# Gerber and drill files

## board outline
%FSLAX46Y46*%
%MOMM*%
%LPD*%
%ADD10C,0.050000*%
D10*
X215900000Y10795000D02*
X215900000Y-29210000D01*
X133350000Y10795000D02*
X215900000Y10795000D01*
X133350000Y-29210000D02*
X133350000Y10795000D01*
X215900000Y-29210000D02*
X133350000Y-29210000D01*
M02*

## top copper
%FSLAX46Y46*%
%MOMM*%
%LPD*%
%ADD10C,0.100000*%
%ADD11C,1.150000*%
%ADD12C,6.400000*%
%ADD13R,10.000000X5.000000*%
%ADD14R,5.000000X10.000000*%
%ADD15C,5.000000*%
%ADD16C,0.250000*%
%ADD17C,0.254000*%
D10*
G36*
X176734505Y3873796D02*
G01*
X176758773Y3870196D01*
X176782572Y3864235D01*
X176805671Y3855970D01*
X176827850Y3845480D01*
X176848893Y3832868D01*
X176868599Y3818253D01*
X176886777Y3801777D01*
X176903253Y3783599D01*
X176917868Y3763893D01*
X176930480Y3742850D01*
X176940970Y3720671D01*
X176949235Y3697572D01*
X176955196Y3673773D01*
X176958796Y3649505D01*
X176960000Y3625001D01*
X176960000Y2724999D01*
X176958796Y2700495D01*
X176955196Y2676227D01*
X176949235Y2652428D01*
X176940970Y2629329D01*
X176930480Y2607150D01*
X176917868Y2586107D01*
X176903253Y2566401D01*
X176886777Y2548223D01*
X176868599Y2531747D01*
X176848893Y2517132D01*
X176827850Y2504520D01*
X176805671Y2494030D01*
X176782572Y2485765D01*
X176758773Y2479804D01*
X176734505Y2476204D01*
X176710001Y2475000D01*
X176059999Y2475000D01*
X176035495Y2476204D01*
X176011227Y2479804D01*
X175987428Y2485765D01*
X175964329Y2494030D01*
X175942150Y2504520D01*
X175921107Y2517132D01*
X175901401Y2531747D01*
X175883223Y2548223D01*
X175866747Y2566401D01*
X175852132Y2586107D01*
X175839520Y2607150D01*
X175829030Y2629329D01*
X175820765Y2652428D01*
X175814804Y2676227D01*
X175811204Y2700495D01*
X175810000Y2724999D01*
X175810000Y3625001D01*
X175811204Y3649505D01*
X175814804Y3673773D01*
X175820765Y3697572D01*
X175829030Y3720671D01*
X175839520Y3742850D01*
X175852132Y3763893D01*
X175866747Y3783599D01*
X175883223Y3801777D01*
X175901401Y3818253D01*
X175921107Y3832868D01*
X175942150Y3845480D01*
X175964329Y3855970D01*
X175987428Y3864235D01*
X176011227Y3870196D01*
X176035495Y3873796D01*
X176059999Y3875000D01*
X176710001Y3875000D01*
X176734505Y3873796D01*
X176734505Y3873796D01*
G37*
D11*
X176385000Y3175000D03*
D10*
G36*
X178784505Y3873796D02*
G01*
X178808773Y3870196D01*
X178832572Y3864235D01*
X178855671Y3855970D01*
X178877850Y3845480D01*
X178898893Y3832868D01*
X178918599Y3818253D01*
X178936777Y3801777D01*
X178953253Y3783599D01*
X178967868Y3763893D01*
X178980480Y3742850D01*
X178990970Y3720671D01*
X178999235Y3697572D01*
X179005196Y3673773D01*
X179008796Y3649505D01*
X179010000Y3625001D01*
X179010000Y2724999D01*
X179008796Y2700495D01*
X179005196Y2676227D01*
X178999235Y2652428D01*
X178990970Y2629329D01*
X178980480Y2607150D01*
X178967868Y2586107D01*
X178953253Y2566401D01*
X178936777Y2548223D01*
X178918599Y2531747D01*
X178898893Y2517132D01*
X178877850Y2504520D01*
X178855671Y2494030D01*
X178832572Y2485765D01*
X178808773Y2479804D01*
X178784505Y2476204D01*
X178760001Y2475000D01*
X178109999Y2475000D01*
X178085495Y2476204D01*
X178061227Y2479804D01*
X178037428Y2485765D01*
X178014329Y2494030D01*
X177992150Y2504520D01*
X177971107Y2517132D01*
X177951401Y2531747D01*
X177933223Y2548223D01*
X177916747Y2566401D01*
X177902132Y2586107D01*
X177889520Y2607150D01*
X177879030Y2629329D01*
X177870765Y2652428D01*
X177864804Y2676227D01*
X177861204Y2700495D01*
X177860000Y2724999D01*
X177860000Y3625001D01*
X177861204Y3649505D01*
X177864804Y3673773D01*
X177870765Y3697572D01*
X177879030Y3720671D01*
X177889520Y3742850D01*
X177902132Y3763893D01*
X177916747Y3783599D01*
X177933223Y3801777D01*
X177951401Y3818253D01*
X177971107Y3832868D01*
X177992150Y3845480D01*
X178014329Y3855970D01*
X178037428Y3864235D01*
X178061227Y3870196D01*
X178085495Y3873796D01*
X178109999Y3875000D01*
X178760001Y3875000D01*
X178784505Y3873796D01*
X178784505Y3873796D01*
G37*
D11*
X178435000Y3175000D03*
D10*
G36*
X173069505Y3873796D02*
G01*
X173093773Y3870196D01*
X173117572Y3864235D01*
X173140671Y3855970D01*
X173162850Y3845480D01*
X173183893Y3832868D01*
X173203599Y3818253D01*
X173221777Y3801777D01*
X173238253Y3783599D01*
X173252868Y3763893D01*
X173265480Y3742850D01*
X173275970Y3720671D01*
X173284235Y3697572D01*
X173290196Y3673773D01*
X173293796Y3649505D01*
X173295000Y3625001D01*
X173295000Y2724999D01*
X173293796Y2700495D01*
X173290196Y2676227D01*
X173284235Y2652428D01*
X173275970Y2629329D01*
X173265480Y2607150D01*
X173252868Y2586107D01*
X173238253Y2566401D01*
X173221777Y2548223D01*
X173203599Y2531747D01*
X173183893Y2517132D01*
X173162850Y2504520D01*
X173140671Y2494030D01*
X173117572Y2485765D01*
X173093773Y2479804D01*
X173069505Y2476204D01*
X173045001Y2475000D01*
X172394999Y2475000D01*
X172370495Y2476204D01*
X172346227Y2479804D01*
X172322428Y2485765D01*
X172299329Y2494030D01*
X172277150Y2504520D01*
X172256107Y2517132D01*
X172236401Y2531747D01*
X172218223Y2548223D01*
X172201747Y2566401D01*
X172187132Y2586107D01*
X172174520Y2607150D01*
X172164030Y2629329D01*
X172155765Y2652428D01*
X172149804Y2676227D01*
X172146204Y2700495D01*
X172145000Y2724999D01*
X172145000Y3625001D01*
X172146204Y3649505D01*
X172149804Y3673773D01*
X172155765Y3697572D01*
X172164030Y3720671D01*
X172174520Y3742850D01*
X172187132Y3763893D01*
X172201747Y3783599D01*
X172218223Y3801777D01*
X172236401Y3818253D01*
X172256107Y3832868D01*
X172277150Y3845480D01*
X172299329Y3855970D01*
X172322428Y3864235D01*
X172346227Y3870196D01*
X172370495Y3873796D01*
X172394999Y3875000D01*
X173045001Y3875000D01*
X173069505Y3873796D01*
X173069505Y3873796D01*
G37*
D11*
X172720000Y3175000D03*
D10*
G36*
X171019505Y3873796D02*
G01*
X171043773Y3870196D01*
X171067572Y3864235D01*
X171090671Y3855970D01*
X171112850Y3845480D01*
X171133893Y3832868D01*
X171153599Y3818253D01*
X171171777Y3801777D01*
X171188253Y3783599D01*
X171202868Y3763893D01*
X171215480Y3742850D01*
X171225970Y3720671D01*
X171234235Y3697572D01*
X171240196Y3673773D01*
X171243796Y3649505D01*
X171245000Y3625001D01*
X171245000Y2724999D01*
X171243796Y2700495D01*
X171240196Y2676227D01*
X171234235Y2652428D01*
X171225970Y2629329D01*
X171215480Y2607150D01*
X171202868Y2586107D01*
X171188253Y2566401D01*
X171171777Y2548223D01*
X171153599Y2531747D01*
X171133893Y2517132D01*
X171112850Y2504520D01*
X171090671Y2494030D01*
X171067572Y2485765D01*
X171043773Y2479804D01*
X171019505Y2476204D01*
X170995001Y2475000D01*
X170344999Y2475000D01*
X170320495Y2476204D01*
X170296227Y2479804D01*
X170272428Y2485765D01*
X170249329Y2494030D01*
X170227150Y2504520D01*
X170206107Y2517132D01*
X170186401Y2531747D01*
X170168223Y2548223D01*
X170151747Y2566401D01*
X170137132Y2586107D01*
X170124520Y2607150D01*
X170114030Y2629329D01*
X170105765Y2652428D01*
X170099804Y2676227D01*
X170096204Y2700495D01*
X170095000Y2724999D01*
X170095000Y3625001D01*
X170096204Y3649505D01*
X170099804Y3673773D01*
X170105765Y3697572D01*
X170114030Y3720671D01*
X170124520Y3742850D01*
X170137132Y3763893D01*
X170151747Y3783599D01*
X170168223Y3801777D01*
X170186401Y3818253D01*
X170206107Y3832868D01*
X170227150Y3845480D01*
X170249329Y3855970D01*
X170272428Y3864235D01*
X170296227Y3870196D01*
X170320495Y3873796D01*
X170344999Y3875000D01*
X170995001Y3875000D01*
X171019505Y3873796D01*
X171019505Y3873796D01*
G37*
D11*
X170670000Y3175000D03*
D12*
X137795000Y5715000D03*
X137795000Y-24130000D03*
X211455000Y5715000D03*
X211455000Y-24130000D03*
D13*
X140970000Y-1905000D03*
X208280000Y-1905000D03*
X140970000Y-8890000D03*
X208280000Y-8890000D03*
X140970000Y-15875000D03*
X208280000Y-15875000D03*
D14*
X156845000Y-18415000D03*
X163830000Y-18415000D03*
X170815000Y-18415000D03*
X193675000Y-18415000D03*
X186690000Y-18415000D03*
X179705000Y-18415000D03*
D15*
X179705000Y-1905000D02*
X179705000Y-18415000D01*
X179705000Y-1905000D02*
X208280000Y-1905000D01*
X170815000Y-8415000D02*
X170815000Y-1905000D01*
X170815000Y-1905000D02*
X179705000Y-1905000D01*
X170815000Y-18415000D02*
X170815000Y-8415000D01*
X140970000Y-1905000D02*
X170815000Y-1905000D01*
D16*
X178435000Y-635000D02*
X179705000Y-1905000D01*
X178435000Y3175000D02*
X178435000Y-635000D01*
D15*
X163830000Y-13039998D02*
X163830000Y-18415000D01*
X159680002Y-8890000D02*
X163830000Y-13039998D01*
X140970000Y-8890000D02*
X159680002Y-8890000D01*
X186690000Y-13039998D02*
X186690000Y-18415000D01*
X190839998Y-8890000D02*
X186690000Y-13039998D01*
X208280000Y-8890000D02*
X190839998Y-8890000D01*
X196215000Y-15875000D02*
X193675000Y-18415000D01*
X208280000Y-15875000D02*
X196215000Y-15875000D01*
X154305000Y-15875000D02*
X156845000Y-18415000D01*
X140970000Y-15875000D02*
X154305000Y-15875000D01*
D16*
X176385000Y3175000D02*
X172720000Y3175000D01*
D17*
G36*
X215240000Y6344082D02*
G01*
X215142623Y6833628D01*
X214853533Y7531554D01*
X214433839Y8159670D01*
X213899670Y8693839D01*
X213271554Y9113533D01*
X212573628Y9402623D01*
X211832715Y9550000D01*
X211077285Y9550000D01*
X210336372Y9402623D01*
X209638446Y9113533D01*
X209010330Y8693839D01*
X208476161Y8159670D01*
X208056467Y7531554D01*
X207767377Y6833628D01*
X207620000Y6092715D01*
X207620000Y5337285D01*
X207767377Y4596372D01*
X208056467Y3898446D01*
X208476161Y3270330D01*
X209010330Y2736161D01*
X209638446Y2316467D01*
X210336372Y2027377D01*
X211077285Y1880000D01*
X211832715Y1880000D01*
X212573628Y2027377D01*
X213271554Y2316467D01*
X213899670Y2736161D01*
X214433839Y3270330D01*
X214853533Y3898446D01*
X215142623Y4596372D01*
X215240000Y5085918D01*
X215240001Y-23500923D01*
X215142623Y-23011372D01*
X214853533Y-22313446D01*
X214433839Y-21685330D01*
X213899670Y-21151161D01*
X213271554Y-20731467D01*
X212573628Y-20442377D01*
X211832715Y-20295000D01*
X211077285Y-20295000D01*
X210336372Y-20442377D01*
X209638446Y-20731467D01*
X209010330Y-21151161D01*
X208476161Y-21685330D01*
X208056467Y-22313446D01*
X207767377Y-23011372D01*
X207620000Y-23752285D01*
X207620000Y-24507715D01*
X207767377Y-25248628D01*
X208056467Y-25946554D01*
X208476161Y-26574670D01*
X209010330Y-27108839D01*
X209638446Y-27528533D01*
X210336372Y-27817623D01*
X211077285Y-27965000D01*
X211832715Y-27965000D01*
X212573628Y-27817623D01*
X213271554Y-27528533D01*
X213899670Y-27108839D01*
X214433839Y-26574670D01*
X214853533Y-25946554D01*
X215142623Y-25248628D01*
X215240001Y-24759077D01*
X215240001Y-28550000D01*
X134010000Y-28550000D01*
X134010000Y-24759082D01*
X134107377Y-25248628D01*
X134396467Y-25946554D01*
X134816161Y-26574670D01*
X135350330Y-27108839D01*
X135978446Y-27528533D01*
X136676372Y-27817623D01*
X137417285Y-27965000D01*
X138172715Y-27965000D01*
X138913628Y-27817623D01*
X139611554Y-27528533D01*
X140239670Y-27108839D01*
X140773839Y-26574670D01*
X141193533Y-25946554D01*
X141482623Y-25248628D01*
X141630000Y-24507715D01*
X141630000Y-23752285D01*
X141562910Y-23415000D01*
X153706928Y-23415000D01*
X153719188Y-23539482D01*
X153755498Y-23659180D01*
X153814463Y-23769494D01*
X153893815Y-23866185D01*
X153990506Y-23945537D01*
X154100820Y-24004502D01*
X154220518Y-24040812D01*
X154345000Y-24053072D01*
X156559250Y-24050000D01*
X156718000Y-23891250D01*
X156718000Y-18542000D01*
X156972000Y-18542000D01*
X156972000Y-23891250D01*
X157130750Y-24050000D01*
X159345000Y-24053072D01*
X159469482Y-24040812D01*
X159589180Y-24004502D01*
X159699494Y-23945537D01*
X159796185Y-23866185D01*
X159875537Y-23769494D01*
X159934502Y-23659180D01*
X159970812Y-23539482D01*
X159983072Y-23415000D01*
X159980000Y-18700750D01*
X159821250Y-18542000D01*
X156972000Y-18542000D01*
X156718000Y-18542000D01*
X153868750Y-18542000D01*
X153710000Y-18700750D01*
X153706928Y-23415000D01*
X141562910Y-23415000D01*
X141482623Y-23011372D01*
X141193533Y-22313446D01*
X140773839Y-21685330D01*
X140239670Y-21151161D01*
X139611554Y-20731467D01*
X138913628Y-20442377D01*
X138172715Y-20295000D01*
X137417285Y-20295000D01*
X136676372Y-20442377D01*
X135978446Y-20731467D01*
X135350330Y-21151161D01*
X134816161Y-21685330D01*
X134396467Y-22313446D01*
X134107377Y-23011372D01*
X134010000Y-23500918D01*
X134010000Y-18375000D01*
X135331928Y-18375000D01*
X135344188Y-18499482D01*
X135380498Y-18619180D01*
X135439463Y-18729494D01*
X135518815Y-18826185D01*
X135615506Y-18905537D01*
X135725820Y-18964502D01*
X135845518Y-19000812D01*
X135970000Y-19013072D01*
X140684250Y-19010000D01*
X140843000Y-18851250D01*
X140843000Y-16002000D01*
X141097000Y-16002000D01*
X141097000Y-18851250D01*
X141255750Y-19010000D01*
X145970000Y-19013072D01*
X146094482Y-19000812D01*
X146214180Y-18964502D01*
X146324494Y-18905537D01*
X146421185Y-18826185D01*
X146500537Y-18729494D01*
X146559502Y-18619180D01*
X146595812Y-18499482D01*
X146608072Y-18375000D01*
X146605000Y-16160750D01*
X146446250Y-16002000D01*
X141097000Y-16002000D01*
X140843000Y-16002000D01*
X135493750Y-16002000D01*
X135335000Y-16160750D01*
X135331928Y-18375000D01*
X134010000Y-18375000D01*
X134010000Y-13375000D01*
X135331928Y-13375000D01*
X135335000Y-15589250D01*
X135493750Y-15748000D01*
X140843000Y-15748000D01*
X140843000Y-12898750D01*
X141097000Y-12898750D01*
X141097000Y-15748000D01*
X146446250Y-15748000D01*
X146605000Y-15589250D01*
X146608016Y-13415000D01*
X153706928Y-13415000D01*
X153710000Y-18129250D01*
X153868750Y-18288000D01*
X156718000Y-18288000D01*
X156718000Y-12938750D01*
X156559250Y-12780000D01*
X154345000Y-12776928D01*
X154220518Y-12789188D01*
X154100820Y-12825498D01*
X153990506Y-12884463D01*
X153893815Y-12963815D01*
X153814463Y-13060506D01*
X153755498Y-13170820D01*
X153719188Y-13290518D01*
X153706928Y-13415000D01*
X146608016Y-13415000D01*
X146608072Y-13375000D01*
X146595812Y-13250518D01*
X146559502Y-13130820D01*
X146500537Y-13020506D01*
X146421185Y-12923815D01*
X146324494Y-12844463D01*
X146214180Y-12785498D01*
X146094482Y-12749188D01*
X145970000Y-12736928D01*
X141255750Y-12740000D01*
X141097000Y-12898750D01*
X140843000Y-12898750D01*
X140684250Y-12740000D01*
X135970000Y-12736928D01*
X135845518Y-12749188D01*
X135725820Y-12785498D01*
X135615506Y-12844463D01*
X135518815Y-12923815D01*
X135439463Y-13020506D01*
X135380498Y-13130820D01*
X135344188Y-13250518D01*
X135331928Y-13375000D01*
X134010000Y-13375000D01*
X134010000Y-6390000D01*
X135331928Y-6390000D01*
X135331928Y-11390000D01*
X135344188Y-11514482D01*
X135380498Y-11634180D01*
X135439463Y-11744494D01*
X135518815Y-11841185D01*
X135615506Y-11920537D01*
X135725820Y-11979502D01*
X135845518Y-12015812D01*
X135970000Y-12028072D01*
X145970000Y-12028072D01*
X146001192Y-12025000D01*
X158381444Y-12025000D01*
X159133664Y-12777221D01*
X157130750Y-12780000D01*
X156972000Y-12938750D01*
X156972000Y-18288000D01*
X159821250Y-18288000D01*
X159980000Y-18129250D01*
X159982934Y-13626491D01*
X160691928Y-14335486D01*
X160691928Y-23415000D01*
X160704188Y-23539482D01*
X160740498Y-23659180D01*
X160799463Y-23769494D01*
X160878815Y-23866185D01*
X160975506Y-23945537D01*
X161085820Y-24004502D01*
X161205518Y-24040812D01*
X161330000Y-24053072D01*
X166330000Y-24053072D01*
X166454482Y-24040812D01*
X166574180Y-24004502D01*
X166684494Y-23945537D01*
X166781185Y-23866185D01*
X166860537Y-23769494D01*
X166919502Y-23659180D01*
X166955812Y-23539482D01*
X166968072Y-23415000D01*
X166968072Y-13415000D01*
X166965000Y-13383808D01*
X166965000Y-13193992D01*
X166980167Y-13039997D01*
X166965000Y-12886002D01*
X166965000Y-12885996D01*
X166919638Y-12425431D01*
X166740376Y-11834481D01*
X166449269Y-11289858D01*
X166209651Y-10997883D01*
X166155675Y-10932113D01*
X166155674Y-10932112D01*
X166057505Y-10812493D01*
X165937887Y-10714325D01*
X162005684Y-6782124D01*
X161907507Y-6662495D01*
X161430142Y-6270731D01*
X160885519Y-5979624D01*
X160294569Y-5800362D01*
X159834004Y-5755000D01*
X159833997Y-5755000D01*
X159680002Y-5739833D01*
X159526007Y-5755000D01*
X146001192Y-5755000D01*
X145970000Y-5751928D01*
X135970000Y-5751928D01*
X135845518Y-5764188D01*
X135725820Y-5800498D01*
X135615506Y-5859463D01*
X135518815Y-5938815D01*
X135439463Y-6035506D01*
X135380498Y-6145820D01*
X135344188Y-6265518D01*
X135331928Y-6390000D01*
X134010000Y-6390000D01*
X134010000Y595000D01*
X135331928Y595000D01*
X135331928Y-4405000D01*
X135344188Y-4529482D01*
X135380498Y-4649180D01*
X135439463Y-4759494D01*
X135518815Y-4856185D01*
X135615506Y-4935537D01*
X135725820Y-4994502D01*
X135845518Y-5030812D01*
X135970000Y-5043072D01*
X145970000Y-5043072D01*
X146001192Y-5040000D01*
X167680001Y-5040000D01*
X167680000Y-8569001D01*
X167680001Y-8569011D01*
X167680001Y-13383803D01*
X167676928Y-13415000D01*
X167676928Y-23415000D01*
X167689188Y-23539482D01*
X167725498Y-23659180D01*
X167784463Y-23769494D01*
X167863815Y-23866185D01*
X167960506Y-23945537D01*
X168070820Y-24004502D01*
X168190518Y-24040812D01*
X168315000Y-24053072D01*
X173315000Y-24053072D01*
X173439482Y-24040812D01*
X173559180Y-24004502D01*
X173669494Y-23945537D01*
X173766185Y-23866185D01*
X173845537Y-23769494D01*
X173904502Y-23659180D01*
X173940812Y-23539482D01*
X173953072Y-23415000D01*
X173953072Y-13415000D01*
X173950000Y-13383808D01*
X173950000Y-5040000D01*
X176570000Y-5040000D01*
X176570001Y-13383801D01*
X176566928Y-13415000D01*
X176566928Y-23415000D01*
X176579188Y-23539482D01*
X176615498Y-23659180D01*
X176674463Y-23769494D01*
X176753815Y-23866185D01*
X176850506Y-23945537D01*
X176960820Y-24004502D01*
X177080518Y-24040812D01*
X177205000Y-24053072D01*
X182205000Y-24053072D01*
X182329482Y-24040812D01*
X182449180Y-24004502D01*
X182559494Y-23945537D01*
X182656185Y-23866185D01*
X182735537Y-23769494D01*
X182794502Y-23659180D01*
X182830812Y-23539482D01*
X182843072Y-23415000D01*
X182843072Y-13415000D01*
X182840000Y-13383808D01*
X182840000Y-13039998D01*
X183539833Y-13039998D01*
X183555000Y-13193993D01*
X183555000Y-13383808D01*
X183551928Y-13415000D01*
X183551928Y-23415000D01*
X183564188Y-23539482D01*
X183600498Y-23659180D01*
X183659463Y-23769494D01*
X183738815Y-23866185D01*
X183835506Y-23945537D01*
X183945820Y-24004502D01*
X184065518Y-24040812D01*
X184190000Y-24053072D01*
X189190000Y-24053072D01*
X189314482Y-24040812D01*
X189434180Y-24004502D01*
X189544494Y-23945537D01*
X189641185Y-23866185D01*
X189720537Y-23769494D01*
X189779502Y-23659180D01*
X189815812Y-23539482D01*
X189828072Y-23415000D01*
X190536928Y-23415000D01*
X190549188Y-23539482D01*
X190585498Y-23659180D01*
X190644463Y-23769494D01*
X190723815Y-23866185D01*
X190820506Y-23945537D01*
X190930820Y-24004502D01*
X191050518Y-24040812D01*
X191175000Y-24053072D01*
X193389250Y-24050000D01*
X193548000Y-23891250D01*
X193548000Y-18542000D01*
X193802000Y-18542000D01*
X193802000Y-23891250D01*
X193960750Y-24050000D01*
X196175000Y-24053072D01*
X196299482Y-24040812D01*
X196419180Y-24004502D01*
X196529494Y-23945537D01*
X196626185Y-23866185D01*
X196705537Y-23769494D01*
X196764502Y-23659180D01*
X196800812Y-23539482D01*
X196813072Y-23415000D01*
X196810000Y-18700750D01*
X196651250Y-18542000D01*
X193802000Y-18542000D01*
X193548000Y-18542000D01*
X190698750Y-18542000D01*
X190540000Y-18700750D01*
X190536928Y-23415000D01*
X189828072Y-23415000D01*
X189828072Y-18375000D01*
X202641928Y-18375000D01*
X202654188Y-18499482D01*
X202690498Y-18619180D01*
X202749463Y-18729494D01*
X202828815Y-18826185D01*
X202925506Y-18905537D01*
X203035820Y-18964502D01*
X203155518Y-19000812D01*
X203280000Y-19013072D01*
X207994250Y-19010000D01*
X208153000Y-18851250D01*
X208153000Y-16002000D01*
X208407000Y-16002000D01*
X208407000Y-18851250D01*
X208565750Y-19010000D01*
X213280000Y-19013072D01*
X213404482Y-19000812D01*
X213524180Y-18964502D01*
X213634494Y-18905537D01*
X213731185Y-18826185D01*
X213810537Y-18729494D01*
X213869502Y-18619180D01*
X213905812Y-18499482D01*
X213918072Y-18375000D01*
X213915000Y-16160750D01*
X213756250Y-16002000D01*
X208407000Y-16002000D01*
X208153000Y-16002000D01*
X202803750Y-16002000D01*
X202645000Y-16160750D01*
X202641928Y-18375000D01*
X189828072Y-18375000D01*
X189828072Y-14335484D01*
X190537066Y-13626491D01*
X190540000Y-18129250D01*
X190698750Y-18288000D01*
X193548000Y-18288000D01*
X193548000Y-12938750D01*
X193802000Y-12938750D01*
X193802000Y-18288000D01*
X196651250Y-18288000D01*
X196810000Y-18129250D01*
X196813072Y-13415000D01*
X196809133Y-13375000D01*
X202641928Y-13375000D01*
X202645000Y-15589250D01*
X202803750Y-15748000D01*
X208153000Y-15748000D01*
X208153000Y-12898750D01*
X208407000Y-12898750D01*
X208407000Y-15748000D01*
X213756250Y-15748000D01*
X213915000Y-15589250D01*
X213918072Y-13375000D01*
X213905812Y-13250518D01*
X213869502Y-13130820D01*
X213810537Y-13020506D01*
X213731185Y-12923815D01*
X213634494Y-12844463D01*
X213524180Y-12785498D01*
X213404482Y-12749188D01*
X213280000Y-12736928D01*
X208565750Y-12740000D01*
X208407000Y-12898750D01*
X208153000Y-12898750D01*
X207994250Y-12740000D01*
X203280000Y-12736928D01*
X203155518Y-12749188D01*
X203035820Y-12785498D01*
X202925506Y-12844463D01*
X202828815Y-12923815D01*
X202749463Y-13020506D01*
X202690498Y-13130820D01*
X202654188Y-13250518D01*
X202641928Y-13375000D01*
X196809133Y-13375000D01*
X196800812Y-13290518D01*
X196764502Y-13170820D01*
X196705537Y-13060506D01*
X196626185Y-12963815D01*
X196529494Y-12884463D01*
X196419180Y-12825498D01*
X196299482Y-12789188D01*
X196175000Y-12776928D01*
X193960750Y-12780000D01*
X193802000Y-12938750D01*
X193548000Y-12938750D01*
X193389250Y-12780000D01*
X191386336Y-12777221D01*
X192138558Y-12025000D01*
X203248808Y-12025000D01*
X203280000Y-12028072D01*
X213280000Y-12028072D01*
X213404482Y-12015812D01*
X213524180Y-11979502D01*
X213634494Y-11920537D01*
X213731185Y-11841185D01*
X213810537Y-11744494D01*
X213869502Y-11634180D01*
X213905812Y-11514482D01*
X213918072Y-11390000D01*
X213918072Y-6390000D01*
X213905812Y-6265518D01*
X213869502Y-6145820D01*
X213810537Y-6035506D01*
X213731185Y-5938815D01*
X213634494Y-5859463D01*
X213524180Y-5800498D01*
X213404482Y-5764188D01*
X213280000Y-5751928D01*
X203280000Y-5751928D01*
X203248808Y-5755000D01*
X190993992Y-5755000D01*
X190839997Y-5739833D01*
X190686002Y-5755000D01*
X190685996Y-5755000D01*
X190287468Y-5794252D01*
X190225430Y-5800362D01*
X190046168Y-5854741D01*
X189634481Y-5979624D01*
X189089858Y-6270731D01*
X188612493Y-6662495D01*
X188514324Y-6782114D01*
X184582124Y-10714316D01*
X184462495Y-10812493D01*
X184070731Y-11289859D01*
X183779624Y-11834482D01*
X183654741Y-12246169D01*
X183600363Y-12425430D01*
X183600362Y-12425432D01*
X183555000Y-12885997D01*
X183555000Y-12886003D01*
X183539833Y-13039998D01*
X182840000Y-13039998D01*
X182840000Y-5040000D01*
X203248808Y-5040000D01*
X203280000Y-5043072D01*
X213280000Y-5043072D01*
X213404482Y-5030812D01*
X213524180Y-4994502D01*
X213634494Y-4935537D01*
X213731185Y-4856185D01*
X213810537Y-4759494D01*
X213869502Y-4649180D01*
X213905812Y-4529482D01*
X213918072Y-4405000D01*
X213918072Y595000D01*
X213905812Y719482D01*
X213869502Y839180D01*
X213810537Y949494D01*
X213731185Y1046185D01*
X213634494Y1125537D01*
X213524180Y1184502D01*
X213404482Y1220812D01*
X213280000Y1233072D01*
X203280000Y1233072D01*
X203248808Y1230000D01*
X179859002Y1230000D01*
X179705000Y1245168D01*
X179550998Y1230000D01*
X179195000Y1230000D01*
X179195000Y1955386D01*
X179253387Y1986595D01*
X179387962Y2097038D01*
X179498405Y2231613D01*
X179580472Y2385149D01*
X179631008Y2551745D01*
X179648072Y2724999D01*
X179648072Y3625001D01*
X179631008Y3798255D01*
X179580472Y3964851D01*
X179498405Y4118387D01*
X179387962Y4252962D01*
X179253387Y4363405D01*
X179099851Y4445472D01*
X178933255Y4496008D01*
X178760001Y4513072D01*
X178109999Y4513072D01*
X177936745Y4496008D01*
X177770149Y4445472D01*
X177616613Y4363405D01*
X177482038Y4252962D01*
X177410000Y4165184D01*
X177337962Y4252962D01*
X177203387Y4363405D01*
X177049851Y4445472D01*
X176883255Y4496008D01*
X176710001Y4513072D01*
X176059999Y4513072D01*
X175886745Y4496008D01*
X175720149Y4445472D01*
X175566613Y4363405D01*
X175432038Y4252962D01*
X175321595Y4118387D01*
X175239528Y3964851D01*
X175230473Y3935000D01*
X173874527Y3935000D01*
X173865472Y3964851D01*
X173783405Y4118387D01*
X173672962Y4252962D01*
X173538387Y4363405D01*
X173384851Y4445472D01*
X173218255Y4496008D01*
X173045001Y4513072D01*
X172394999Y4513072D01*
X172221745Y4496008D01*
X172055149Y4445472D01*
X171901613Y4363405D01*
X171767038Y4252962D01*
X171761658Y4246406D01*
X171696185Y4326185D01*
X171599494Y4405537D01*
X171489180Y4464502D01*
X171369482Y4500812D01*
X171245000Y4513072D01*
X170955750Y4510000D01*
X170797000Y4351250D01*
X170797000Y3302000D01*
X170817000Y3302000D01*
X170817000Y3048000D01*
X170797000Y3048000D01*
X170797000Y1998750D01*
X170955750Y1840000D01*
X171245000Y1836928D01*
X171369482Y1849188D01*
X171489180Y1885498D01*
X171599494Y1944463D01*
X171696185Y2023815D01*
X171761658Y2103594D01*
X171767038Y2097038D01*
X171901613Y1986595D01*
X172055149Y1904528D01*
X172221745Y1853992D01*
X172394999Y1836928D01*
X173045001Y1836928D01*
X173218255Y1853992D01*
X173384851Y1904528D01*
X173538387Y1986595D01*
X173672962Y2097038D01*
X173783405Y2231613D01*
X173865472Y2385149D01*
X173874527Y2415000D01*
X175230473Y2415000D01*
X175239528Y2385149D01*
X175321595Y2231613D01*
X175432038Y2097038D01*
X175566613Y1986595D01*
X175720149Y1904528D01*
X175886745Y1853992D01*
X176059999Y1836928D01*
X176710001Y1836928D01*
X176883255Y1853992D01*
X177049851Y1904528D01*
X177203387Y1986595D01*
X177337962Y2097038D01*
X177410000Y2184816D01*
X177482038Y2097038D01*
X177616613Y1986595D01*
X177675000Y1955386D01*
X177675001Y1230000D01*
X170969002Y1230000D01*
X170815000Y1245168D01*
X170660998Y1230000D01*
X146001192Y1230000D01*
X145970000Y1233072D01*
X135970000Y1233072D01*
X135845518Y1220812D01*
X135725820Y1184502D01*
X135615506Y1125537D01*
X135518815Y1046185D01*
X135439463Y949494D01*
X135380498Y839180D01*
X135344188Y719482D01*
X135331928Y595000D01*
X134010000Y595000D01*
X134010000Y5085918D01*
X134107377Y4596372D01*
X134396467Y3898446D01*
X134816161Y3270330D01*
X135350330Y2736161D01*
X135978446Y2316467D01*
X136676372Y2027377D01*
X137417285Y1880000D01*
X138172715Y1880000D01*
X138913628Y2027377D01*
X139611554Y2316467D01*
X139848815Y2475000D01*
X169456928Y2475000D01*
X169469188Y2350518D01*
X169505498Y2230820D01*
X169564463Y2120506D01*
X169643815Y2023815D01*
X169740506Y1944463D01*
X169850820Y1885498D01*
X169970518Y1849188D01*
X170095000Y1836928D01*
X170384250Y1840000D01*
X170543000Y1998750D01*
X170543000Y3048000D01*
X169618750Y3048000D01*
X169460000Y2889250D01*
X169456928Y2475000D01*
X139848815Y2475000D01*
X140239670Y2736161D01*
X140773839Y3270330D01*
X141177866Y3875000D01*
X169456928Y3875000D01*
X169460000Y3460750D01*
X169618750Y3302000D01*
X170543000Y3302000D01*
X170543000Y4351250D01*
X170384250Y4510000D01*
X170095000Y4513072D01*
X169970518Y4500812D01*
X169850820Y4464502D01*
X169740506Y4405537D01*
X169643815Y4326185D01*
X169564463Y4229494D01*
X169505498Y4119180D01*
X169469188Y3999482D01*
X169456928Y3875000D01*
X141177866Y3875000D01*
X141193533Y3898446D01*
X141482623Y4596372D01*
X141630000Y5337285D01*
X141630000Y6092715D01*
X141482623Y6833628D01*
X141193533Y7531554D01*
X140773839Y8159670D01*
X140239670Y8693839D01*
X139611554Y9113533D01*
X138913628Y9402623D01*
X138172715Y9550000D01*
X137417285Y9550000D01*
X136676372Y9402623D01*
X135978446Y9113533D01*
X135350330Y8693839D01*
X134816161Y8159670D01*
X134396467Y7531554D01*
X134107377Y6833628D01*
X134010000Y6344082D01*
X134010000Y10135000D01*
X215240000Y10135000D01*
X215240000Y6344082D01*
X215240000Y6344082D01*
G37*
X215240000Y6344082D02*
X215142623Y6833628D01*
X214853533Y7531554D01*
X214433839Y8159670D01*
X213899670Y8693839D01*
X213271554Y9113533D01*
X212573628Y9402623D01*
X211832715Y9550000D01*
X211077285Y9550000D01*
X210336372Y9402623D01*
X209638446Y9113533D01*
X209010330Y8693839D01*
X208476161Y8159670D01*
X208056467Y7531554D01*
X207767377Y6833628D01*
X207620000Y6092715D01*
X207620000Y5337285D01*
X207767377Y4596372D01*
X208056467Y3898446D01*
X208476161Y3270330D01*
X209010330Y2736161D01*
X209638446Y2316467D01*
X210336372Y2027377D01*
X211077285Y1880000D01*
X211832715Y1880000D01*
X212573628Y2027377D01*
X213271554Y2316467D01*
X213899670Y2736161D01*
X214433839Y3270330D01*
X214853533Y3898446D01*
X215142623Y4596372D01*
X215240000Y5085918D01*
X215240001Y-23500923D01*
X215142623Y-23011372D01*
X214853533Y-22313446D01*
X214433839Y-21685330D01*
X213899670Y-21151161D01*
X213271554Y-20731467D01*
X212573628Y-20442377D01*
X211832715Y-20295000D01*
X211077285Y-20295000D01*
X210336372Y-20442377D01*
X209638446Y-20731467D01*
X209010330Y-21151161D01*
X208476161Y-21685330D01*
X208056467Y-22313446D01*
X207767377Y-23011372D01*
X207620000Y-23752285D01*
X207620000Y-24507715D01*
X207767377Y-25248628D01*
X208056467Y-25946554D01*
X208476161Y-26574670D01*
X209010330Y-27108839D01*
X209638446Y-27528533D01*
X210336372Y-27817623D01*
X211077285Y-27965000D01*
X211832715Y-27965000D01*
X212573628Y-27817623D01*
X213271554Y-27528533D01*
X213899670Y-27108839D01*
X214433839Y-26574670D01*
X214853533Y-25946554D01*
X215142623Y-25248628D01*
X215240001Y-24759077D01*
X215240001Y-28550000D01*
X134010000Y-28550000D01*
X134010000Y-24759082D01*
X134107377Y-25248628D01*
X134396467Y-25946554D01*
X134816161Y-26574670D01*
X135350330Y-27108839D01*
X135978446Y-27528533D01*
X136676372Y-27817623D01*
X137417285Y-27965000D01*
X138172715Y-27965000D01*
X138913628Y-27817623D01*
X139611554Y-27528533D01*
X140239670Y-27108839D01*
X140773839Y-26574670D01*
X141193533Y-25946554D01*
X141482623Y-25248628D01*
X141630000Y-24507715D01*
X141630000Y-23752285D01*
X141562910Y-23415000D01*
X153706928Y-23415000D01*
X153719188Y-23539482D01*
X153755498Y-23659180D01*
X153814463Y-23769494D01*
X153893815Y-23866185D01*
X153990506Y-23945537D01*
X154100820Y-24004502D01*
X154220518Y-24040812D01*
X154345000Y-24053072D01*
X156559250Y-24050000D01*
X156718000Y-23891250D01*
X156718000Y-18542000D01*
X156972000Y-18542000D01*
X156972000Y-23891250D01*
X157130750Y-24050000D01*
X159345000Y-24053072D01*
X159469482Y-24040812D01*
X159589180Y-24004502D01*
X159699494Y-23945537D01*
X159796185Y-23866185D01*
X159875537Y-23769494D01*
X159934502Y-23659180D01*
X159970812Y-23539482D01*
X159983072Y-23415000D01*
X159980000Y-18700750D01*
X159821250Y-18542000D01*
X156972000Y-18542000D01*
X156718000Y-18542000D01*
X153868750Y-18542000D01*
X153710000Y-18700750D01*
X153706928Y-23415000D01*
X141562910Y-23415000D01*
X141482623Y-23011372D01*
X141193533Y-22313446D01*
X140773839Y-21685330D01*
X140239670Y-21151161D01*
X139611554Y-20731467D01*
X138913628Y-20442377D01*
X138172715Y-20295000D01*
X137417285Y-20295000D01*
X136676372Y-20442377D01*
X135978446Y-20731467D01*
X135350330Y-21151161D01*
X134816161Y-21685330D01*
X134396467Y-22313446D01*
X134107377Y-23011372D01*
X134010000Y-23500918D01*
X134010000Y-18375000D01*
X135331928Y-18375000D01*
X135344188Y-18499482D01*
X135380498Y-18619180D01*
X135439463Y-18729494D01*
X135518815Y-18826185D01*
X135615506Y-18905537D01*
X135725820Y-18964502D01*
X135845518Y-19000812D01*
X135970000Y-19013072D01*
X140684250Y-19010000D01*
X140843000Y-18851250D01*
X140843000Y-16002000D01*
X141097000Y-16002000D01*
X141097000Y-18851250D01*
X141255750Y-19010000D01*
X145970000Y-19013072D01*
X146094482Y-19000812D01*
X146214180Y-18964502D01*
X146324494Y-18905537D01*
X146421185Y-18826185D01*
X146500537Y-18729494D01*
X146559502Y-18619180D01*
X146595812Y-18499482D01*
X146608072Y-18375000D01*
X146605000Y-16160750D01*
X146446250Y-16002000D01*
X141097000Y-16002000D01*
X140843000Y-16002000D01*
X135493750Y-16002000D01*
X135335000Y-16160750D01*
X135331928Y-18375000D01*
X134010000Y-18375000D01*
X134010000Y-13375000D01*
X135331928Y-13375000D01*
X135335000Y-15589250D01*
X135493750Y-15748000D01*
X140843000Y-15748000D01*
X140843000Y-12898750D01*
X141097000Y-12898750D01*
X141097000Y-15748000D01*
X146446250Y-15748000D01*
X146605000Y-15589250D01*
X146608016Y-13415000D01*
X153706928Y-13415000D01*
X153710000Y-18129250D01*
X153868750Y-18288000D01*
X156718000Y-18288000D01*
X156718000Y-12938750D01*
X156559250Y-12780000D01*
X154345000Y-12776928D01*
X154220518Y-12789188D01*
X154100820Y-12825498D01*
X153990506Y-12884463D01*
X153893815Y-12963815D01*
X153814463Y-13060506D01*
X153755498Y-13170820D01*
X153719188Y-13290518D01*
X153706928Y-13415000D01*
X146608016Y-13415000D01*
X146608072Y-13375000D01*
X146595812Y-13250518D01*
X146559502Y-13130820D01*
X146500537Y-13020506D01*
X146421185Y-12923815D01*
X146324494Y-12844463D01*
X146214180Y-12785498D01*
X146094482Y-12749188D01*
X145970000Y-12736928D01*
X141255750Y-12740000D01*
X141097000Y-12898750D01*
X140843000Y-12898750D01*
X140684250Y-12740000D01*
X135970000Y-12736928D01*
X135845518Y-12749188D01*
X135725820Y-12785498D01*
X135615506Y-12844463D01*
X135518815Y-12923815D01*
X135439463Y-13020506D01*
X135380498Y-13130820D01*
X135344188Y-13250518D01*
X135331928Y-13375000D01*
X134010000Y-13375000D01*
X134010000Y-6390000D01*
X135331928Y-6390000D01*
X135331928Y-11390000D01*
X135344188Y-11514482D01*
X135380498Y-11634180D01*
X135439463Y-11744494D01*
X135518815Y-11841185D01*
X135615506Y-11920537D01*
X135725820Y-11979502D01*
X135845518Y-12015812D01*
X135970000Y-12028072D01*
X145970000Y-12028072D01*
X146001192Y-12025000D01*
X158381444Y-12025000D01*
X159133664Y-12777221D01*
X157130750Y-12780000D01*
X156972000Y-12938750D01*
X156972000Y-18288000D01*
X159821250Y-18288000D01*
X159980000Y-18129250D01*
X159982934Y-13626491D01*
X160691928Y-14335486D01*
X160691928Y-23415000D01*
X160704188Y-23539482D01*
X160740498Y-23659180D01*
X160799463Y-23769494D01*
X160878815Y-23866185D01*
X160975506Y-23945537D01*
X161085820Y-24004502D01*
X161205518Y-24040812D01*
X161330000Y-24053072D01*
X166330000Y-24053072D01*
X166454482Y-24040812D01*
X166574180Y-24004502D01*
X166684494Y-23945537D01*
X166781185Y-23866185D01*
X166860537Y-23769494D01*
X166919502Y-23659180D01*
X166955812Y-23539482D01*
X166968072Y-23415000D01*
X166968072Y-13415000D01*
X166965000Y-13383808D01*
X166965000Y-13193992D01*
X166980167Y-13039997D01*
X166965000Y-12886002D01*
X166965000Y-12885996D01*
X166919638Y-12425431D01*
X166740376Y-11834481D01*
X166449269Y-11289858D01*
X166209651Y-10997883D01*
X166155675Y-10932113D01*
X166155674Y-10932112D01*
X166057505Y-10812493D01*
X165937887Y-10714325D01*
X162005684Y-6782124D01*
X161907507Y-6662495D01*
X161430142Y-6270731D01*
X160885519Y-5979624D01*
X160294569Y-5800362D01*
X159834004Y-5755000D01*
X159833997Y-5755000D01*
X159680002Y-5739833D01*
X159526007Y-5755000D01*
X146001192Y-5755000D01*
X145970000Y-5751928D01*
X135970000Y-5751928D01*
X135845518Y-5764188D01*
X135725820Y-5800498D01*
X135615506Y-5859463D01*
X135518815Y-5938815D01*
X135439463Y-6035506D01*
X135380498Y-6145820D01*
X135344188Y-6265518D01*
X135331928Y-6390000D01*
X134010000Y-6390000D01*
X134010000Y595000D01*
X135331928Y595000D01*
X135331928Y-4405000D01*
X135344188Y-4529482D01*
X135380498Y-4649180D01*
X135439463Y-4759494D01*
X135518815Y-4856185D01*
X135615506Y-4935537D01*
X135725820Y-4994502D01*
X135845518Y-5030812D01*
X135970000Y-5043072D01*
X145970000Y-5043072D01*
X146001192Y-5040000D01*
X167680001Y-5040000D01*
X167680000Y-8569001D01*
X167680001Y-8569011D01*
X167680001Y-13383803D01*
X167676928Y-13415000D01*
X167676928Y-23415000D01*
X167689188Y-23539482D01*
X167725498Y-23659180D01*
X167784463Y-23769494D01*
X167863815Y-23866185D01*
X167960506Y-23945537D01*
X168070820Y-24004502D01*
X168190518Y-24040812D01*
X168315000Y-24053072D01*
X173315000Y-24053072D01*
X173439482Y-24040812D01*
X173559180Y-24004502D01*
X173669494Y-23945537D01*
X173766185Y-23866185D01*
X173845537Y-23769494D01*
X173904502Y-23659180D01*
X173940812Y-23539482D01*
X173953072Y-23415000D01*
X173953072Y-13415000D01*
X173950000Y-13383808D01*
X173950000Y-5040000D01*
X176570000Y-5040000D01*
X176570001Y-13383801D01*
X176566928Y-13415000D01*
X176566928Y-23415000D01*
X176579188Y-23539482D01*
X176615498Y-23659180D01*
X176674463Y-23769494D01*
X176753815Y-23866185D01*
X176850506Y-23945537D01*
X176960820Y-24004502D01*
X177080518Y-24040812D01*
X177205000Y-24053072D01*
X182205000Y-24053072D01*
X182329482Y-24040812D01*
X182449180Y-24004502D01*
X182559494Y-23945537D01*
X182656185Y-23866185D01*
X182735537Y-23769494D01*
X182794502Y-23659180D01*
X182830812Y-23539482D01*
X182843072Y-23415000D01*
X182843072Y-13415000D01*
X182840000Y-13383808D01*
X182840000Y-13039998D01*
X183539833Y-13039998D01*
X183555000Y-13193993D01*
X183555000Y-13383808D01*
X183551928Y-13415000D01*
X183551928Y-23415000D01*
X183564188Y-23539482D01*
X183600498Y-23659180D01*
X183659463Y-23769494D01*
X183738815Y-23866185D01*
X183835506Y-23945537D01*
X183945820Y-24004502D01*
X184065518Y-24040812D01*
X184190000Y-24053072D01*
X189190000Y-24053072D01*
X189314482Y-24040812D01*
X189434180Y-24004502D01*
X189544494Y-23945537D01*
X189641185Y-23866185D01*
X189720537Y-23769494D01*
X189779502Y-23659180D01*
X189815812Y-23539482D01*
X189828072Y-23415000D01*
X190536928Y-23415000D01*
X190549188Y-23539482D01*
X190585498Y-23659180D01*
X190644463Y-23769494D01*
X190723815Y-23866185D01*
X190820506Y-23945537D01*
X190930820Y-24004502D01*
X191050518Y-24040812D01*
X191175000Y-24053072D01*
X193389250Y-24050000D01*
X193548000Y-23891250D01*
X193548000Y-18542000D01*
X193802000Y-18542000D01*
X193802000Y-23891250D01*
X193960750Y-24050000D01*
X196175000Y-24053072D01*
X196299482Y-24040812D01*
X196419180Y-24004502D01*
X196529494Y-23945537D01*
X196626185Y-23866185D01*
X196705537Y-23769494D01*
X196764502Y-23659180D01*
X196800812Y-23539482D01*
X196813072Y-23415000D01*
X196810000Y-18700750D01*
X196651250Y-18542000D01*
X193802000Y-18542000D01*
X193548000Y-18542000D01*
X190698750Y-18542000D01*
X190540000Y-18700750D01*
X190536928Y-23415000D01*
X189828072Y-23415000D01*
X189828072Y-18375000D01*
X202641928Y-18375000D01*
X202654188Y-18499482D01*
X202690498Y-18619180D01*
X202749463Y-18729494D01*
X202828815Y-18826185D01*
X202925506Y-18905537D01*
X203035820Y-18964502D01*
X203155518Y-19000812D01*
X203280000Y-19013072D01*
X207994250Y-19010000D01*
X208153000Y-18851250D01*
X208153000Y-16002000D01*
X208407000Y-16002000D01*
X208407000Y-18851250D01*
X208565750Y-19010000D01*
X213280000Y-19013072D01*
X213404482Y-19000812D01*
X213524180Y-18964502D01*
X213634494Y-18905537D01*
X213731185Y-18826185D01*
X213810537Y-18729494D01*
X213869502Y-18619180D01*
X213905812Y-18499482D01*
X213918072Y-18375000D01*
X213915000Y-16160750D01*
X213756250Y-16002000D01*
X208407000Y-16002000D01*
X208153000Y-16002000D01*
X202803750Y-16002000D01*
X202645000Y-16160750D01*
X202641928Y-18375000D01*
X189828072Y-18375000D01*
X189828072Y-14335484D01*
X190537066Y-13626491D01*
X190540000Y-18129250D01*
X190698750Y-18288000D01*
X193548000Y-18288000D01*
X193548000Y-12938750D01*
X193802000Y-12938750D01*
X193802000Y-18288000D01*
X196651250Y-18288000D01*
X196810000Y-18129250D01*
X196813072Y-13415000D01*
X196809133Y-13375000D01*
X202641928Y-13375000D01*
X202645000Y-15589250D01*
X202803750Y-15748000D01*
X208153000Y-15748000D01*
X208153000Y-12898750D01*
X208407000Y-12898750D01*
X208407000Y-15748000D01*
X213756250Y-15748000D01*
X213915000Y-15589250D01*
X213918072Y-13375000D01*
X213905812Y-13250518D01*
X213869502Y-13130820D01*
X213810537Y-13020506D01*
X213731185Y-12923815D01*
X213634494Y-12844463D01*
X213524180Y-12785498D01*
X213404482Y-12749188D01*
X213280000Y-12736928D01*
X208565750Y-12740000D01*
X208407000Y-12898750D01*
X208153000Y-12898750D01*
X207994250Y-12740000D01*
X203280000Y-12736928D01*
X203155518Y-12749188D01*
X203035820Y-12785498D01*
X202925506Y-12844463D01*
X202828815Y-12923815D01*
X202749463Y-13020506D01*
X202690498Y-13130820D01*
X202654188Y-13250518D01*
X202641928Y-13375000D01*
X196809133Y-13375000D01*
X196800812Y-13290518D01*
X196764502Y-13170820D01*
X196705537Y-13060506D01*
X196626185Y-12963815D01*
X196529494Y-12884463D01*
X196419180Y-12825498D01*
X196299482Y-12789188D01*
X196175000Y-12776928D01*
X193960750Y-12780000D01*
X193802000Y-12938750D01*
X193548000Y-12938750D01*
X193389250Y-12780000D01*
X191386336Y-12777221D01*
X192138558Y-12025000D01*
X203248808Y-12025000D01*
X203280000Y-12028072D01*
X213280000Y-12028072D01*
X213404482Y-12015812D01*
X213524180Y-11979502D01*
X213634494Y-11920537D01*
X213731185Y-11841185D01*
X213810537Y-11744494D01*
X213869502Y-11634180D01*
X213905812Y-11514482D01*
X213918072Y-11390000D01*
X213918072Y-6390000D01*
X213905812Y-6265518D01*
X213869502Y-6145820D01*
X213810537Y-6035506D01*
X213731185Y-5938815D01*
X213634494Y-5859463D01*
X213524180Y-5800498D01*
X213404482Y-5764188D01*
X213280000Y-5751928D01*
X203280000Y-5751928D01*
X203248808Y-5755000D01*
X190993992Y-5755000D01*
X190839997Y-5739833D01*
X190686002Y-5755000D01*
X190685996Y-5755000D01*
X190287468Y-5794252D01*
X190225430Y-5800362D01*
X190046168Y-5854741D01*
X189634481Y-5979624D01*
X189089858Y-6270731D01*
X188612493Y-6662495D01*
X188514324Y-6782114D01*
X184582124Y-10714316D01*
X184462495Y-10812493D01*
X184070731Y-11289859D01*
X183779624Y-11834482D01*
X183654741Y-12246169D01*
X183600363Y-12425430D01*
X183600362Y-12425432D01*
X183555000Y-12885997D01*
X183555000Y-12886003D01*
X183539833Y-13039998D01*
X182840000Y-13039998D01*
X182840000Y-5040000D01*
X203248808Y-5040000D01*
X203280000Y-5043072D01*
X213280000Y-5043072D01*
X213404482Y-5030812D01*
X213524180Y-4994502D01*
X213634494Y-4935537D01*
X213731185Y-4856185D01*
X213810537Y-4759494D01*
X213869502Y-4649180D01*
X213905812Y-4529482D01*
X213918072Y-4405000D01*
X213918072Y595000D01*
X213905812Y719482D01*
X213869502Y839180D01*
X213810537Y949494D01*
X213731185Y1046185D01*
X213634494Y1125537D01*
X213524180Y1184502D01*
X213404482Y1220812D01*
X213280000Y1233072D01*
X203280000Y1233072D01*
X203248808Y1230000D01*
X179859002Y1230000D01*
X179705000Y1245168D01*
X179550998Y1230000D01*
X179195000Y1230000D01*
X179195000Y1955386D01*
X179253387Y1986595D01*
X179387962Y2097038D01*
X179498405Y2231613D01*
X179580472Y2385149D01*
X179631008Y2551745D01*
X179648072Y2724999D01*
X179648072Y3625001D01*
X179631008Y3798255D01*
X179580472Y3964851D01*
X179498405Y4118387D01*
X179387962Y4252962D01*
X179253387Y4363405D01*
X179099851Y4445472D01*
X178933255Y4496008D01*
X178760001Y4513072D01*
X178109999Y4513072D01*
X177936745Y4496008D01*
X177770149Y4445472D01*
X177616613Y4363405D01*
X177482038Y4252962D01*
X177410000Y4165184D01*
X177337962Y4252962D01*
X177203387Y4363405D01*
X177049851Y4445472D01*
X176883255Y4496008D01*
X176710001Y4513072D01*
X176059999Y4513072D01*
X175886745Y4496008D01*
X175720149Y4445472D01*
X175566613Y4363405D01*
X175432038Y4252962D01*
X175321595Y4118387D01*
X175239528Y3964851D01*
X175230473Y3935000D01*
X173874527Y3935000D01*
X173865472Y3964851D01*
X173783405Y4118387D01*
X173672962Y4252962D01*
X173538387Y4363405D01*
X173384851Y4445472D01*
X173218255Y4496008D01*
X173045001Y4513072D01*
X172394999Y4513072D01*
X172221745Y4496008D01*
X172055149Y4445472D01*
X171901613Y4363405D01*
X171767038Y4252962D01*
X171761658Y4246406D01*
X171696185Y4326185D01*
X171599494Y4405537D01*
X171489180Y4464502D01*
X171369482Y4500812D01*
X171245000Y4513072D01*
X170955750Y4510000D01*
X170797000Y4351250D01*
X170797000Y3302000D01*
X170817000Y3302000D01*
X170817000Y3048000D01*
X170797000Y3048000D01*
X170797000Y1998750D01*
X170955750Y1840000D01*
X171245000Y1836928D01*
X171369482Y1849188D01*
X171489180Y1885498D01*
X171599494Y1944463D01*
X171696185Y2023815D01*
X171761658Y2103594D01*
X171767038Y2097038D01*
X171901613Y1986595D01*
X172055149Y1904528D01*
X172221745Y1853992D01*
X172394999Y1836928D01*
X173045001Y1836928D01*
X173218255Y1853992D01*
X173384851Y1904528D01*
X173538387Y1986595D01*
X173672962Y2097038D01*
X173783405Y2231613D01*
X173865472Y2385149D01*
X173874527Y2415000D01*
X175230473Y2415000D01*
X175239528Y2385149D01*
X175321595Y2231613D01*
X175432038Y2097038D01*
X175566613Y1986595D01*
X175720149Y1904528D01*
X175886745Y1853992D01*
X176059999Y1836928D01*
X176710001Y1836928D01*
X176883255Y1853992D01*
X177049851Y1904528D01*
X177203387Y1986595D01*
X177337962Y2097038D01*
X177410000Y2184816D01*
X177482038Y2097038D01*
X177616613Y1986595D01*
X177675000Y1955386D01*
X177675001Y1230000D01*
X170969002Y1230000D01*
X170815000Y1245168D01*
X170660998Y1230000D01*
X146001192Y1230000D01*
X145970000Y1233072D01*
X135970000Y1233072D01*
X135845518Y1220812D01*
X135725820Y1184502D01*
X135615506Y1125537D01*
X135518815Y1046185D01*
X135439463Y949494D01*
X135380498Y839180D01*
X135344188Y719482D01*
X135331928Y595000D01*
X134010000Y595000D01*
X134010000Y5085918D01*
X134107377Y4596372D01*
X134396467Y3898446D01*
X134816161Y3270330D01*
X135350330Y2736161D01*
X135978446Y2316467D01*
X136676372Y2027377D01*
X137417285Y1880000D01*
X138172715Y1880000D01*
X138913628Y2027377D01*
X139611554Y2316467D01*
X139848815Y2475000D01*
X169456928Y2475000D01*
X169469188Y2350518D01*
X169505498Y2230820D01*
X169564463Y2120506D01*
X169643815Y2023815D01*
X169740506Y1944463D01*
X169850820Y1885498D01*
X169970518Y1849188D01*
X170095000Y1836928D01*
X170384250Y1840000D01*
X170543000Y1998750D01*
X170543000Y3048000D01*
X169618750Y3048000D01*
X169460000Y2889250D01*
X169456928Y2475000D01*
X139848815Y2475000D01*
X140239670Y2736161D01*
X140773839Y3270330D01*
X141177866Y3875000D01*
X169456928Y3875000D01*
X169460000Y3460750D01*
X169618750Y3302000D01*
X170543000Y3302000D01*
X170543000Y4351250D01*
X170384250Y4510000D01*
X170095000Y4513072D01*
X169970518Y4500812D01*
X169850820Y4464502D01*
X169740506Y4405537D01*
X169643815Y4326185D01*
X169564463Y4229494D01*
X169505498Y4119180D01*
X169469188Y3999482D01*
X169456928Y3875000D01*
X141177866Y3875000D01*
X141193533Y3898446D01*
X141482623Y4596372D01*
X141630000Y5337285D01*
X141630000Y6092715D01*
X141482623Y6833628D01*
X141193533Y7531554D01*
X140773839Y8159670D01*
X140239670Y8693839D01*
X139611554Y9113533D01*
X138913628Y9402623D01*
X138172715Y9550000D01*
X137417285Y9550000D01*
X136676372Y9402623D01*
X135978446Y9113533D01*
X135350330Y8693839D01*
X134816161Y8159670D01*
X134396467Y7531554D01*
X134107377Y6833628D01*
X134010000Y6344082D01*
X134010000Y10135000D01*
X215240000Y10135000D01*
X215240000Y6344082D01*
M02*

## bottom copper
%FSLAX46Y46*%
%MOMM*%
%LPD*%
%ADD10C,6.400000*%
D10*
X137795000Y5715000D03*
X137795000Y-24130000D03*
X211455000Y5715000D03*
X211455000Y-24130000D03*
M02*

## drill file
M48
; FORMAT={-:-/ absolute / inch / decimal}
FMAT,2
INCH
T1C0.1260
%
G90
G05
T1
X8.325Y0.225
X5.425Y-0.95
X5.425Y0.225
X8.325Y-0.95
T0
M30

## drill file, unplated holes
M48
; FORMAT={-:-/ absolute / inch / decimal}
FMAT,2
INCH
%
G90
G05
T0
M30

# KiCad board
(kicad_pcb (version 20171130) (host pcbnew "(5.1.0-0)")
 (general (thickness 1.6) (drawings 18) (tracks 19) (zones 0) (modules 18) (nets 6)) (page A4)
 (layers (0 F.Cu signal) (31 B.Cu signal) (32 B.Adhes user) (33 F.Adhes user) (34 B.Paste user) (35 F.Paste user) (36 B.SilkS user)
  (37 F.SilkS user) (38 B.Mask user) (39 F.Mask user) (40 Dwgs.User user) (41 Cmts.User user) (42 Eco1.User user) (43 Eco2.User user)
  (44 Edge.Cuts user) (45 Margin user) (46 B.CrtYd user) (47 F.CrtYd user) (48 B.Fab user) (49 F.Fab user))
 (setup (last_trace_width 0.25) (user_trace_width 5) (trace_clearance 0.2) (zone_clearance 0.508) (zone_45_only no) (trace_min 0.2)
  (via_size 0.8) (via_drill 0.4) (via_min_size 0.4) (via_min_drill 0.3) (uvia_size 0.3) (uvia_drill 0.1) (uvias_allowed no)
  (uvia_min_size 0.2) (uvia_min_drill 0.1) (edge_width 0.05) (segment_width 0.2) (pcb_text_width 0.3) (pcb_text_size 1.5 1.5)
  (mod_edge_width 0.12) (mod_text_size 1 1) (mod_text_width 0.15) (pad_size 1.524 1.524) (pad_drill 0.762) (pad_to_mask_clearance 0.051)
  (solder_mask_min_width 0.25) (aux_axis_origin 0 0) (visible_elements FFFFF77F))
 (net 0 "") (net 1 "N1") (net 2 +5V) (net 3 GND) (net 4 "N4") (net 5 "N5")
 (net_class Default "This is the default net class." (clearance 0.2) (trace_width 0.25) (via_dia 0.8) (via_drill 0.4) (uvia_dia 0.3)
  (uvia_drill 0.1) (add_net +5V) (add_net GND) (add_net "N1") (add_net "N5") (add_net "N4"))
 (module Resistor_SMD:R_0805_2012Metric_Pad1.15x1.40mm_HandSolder (layer F.Cu) (at 177.41 -3.175 180)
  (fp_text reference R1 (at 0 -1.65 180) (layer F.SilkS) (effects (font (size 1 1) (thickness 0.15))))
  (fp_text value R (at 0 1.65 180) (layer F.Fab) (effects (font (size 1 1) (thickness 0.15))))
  (pad 2 smd roundrect (at 1.025 0 180) (size 1.15 1.4) (layers F.Cu F.Paste F.Mask) (roundrect_rratio 0.217391) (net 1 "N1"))
  (pad 1 smd roundrect (at -1.025 0 180) (size 1.15 1.4) (layers F.Cu F.Paste F.Mask) (roundrect_rratio 0.217391) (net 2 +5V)))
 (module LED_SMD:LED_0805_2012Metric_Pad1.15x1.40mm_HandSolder (layer F.Cu) (at 171.695 -3.175)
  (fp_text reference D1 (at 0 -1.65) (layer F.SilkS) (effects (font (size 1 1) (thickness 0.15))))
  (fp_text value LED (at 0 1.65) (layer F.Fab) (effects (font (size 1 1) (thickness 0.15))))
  (pad 2 smd roundrect (at 1.025 0) (size 1.15 1.4) (layers F.Cu F.Paste F.Mask) (roundrect_rratio 0.217391) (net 1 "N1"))
  (pad 1 smd roundrect (at -1.025 0) (size 1.15 1.4) (layers F.Cu F.Paste F.Mask) (roundrect_rratio 0.217391) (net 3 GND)))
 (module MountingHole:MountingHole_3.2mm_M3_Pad (layer F.Cu) (at 137.795 -5.715)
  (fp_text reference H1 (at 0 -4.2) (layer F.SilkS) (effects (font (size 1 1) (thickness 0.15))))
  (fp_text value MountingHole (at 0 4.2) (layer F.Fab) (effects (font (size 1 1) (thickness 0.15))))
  (pad 1 thru_hole circle (at 0 0) (size 6.4 6.4) (drill 3.2) (layers *.Cu *.Mask)))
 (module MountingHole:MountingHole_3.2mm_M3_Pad (layer F.Cu) (at 137.795 24.13)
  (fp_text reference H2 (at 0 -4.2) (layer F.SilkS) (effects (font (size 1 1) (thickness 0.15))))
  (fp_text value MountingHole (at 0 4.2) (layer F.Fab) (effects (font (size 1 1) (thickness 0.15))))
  (pad 1 thru_hole circle (at 0 0) (size 6.4 6.4) (drill 3.2) (layers *.Cu *.Mask)))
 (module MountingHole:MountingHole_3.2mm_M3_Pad (layer F.Cu) (at 211.455 -5.715)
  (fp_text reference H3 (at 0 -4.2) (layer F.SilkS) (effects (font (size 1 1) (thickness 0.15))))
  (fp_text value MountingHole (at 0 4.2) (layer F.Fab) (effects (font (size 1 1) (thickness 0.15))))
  (pad 1 thru_hole circle (at 0 0) (size 6.4 6.4) (drill 3.2) (layers *.Cu *.Mask)))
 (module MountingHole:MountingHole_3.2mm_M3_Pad (layer F.Cu) (at 211.455 24.13)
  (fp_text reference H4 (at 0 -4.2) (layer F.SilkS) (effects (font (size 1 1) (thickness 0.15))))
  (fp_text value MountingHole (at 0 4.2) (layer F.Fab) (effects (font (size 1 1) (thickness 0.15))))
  (pad 1 thru_hole circle (at 0 0) (size 6.4 6.4) (drill 3.2) (layers *.Cu *.Mask)))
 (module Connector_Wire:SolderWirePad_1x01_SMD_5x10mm (layer F.Cu) (at 140.97 1.905 90)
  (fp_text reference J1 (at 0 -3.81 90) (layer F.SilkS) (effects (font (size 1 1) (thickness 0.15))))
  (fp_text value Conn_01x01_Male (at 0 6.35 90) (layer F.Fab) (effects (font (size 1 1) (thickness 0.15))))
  (pad 1 smd rect (at 0 0 90) (size 5 10) (layers F.Cu F.Paste F.Mask) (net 2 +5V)))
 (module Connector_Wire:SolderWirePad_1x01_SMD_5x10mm (layer F.Cu) (at 208.28 1.905 90)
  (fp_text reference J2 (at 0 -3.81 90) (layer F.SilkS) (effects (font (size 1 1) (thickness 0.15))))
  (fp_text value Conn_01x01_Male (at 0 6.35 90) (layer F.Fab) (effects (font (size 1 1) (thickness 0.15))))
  (pad 1 smd rect (at 0 0 90) (size 5 10) (layers F.Cu F.Paste F.Mask) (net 2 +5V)))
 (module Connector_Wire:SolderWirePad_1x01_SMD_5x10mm (layer F.Cu) (at 140.97 8.89 90)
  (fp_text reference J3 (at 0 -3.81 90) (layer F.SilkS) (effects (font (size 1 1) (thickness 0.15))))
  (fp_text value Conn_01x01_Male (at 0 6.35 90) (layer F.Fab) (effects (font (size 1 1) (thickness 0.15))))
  (pad 1 smd rect (at 0 0 90) (size 5 10) (layers F.Cu F.Paste F.Mask) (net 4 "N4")))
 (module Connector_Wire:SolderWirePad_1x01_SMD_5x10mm (layer F.Cu) (at 208.28 8.89 90)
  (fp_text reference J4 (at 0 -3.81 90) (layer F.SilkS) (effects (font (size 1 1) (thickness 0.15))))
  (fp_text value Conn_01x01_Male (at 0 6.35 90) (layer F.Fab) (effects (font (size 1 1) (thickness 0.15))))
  (pad 1 smd rect (at 0 0 90) (size 5 10) (layers F.Cu F.Paste F.Mask) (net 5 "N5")))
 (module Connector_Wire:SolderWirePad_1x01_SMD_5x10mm (layer F.Cu) (at 140.97 15.875 90)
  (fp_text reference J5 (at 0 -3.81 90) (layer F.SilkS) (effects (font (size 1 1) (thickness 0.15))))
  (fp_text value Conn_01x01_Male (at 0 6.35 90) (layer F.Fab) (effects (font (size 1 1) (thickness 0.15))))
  (pad 1 smd rect (at 0 0 90) (size 5 10) (layers F.Cu F.Paste F.Mask) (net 3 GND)))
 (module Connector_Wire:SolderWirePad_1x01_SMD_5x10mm (layer F.Cu) (at 208.28 15.875 90)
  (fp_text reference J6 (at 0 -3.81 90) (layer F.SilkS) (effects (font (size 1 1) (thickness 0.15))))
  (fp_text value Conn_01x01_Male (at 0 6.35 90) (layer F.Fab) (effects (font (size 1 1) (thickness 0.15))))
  (pad 1 smd rect (at 0 0 90) (size 5 10) (layers F.Cu F.Paste F.Mask) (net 3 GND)))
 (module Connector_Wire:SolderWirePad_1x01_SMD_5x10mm (layer F.Cu) (at 156.845 18.415)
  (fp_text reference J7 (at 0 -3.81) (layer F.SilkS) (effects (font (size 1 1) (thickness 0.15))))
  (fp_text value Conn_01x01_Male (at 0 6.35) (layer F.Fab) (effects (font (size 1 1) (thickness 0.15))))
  (pad 1 smd rect (at 0 0) (size 5 10) (layers F.Cu F.Paste F.Mask) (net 3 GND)))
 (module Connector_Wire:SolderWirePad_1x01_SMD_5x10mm (layer F.Cu) (at 163.83 18.415)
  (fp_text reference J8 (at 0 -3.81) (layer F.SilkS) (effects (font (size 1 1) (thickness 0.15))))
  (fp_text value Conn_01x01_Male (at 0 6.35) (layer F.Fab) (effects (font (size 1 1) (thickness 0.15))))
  (pad 1 smd rect (at 0 0) (size 5 10) (layers F.Cu F.Paste F.Mask) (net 4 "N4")))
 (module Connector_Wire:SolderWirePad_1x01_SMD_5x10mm (layer F.Cu) (at 170.815 18.415)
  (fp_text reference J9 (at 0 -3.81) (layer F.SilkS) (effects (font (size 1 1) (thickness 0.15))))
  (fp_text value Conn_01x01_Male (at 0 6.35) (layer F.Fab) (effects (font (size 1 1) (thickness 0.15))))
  (pad 1 smd rect (at 0 0) (size 5 10) (layers F.Cu F.Paste F.Mask) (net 2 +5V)))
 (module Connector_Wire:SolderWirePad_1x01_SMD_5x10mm (layer F.Cu) (at 193.675 18.415)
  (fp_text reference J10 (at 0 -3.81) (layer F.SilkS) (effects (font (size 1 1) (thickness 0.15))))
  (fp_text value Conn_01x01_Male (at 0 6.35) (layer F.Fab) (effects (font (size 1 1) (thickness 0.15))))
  (pad 1 smd rect (at 0 0) (size 5 10) (layers F.Cu F.Paste F.Mask) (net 3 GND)))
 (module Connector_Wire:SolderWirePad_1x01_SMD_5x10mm (layer F.Cu) (at 186.69 18.415)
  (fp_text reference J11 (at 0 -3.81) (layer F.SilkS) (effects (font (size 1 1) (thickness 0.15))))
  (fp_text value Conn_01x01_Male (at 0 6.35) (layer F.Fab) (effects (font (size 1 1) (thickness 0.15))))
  (pad 1 smd rect (at 0 0) (size 5 10) (layers F.Cu F.Paste F.Mask) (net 5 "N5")))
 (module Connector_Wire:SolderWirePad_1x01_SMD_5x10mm (layer F.Cu) (at 179.705 18.415)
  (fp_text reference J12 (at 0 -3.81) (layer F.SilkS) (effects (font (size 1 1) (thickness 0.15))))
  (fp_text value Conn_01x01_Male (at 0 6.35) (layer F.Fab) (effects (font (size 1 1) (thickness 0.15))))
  (pad 1 smd rect (at 0 0) (size 5 10) (layers F.Cu F.Paste F.Mask) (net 2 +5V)))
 (gr_line (start 215.9 -10.795) (end 215.9 29.21) (layer Edge.Cuts) (width 0.05))
 (gr_line (start 133.35 -10.795) (end 215.9 -10.795) (layer Edge.Cuts) (width 0.05))
 (gr_line (start 133.35 29.21) (end 133.35 -10.795) (layer Edge.Cuts) (width 0.05))
 (gr_line (start 215.9 29.21) (end 133.35 29.21) (layer Edge.Cuts) (width 0.05))
 (segment (start 179.705 1.905) (end 179.705 18.415) (width 5) (layer F.Cu) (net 2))
 (segment (start 179.705 1.905) (end 208.28 1.905) (width 5) (layer F.Cu) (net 2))
 (segment (start 170.815 8.415) (end 170.815 1.905) (width 5) (layer F.Cu) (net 2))
 (segment (start 170.815 1.905) (end 179.705 1.905) (width 5) (layer F.Cu) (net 2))
 (segment (start 170.815 18.415) (end 170.815 8.415) (width 5) (layer F.Cu) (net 2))
 (segment (start 140.97 1.905) (end 170.815 1.905) (width 5) (layer F.Cu) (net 2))
 (segment (start 178.435 0.635) (end 179.705 1.905) (width 0.25) (layer F.Cu) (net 2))
 (segment (start 178.435 -3.175) (end 178.435 0.635) (width 0.25) (layer F.Cu) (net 2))
 (segment (start 163.83 13.039998) (end 163.83 18.415) (width 5) (layer F.Cu) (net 4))
 (segment (start 159.680002 8.89) (end 163.83 13.039998) (width 5) (layer F.Cu) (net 4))
 (segment (start 140.97 8.89) (end 159.680002 8.89) (width 5) (layer F.Cu) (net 4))
 (segment (start 186.69 13.039998) (end 186.69 18.415) (width 5) (layer F.Cu) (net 5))
 (segment (start 190.839998 8.89) (end 186.69 13.039998) (width 5) (layer F.Cu) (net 5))
 (segment (start 208.28 8.89) (end 190.839998 8.89) (width 5) (layer F.Cu) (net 5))
 (segment (start 196.215 15.875) (end 193.675 18.415) (width 5) (layer F.Cu) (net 3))
 (segment (start 208.28 15.875) (end 196.215 15.875) (width 5) (layer F.Cu) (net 3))
 (segment (start 154.305 15.875) (end 156.845 18.415) (width 5) (layer F.Cu) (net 3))
 (segment (start 140.97 15.875) (end 154.305 15.875) (width 5) (layer F.Cu) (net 3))
 (segment (start 176.385 -3.175) (end 172.72 -3.175) (width 0.25) (layer F.Cu) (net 1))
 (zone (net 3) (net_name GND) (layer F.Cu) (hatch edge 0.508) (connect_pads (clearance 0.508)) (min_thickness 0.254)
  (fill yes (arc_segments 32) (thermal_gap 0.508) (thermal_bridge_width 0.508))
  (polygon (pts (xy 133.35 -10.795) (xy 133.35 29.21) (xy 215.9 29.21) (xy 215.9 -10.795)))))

